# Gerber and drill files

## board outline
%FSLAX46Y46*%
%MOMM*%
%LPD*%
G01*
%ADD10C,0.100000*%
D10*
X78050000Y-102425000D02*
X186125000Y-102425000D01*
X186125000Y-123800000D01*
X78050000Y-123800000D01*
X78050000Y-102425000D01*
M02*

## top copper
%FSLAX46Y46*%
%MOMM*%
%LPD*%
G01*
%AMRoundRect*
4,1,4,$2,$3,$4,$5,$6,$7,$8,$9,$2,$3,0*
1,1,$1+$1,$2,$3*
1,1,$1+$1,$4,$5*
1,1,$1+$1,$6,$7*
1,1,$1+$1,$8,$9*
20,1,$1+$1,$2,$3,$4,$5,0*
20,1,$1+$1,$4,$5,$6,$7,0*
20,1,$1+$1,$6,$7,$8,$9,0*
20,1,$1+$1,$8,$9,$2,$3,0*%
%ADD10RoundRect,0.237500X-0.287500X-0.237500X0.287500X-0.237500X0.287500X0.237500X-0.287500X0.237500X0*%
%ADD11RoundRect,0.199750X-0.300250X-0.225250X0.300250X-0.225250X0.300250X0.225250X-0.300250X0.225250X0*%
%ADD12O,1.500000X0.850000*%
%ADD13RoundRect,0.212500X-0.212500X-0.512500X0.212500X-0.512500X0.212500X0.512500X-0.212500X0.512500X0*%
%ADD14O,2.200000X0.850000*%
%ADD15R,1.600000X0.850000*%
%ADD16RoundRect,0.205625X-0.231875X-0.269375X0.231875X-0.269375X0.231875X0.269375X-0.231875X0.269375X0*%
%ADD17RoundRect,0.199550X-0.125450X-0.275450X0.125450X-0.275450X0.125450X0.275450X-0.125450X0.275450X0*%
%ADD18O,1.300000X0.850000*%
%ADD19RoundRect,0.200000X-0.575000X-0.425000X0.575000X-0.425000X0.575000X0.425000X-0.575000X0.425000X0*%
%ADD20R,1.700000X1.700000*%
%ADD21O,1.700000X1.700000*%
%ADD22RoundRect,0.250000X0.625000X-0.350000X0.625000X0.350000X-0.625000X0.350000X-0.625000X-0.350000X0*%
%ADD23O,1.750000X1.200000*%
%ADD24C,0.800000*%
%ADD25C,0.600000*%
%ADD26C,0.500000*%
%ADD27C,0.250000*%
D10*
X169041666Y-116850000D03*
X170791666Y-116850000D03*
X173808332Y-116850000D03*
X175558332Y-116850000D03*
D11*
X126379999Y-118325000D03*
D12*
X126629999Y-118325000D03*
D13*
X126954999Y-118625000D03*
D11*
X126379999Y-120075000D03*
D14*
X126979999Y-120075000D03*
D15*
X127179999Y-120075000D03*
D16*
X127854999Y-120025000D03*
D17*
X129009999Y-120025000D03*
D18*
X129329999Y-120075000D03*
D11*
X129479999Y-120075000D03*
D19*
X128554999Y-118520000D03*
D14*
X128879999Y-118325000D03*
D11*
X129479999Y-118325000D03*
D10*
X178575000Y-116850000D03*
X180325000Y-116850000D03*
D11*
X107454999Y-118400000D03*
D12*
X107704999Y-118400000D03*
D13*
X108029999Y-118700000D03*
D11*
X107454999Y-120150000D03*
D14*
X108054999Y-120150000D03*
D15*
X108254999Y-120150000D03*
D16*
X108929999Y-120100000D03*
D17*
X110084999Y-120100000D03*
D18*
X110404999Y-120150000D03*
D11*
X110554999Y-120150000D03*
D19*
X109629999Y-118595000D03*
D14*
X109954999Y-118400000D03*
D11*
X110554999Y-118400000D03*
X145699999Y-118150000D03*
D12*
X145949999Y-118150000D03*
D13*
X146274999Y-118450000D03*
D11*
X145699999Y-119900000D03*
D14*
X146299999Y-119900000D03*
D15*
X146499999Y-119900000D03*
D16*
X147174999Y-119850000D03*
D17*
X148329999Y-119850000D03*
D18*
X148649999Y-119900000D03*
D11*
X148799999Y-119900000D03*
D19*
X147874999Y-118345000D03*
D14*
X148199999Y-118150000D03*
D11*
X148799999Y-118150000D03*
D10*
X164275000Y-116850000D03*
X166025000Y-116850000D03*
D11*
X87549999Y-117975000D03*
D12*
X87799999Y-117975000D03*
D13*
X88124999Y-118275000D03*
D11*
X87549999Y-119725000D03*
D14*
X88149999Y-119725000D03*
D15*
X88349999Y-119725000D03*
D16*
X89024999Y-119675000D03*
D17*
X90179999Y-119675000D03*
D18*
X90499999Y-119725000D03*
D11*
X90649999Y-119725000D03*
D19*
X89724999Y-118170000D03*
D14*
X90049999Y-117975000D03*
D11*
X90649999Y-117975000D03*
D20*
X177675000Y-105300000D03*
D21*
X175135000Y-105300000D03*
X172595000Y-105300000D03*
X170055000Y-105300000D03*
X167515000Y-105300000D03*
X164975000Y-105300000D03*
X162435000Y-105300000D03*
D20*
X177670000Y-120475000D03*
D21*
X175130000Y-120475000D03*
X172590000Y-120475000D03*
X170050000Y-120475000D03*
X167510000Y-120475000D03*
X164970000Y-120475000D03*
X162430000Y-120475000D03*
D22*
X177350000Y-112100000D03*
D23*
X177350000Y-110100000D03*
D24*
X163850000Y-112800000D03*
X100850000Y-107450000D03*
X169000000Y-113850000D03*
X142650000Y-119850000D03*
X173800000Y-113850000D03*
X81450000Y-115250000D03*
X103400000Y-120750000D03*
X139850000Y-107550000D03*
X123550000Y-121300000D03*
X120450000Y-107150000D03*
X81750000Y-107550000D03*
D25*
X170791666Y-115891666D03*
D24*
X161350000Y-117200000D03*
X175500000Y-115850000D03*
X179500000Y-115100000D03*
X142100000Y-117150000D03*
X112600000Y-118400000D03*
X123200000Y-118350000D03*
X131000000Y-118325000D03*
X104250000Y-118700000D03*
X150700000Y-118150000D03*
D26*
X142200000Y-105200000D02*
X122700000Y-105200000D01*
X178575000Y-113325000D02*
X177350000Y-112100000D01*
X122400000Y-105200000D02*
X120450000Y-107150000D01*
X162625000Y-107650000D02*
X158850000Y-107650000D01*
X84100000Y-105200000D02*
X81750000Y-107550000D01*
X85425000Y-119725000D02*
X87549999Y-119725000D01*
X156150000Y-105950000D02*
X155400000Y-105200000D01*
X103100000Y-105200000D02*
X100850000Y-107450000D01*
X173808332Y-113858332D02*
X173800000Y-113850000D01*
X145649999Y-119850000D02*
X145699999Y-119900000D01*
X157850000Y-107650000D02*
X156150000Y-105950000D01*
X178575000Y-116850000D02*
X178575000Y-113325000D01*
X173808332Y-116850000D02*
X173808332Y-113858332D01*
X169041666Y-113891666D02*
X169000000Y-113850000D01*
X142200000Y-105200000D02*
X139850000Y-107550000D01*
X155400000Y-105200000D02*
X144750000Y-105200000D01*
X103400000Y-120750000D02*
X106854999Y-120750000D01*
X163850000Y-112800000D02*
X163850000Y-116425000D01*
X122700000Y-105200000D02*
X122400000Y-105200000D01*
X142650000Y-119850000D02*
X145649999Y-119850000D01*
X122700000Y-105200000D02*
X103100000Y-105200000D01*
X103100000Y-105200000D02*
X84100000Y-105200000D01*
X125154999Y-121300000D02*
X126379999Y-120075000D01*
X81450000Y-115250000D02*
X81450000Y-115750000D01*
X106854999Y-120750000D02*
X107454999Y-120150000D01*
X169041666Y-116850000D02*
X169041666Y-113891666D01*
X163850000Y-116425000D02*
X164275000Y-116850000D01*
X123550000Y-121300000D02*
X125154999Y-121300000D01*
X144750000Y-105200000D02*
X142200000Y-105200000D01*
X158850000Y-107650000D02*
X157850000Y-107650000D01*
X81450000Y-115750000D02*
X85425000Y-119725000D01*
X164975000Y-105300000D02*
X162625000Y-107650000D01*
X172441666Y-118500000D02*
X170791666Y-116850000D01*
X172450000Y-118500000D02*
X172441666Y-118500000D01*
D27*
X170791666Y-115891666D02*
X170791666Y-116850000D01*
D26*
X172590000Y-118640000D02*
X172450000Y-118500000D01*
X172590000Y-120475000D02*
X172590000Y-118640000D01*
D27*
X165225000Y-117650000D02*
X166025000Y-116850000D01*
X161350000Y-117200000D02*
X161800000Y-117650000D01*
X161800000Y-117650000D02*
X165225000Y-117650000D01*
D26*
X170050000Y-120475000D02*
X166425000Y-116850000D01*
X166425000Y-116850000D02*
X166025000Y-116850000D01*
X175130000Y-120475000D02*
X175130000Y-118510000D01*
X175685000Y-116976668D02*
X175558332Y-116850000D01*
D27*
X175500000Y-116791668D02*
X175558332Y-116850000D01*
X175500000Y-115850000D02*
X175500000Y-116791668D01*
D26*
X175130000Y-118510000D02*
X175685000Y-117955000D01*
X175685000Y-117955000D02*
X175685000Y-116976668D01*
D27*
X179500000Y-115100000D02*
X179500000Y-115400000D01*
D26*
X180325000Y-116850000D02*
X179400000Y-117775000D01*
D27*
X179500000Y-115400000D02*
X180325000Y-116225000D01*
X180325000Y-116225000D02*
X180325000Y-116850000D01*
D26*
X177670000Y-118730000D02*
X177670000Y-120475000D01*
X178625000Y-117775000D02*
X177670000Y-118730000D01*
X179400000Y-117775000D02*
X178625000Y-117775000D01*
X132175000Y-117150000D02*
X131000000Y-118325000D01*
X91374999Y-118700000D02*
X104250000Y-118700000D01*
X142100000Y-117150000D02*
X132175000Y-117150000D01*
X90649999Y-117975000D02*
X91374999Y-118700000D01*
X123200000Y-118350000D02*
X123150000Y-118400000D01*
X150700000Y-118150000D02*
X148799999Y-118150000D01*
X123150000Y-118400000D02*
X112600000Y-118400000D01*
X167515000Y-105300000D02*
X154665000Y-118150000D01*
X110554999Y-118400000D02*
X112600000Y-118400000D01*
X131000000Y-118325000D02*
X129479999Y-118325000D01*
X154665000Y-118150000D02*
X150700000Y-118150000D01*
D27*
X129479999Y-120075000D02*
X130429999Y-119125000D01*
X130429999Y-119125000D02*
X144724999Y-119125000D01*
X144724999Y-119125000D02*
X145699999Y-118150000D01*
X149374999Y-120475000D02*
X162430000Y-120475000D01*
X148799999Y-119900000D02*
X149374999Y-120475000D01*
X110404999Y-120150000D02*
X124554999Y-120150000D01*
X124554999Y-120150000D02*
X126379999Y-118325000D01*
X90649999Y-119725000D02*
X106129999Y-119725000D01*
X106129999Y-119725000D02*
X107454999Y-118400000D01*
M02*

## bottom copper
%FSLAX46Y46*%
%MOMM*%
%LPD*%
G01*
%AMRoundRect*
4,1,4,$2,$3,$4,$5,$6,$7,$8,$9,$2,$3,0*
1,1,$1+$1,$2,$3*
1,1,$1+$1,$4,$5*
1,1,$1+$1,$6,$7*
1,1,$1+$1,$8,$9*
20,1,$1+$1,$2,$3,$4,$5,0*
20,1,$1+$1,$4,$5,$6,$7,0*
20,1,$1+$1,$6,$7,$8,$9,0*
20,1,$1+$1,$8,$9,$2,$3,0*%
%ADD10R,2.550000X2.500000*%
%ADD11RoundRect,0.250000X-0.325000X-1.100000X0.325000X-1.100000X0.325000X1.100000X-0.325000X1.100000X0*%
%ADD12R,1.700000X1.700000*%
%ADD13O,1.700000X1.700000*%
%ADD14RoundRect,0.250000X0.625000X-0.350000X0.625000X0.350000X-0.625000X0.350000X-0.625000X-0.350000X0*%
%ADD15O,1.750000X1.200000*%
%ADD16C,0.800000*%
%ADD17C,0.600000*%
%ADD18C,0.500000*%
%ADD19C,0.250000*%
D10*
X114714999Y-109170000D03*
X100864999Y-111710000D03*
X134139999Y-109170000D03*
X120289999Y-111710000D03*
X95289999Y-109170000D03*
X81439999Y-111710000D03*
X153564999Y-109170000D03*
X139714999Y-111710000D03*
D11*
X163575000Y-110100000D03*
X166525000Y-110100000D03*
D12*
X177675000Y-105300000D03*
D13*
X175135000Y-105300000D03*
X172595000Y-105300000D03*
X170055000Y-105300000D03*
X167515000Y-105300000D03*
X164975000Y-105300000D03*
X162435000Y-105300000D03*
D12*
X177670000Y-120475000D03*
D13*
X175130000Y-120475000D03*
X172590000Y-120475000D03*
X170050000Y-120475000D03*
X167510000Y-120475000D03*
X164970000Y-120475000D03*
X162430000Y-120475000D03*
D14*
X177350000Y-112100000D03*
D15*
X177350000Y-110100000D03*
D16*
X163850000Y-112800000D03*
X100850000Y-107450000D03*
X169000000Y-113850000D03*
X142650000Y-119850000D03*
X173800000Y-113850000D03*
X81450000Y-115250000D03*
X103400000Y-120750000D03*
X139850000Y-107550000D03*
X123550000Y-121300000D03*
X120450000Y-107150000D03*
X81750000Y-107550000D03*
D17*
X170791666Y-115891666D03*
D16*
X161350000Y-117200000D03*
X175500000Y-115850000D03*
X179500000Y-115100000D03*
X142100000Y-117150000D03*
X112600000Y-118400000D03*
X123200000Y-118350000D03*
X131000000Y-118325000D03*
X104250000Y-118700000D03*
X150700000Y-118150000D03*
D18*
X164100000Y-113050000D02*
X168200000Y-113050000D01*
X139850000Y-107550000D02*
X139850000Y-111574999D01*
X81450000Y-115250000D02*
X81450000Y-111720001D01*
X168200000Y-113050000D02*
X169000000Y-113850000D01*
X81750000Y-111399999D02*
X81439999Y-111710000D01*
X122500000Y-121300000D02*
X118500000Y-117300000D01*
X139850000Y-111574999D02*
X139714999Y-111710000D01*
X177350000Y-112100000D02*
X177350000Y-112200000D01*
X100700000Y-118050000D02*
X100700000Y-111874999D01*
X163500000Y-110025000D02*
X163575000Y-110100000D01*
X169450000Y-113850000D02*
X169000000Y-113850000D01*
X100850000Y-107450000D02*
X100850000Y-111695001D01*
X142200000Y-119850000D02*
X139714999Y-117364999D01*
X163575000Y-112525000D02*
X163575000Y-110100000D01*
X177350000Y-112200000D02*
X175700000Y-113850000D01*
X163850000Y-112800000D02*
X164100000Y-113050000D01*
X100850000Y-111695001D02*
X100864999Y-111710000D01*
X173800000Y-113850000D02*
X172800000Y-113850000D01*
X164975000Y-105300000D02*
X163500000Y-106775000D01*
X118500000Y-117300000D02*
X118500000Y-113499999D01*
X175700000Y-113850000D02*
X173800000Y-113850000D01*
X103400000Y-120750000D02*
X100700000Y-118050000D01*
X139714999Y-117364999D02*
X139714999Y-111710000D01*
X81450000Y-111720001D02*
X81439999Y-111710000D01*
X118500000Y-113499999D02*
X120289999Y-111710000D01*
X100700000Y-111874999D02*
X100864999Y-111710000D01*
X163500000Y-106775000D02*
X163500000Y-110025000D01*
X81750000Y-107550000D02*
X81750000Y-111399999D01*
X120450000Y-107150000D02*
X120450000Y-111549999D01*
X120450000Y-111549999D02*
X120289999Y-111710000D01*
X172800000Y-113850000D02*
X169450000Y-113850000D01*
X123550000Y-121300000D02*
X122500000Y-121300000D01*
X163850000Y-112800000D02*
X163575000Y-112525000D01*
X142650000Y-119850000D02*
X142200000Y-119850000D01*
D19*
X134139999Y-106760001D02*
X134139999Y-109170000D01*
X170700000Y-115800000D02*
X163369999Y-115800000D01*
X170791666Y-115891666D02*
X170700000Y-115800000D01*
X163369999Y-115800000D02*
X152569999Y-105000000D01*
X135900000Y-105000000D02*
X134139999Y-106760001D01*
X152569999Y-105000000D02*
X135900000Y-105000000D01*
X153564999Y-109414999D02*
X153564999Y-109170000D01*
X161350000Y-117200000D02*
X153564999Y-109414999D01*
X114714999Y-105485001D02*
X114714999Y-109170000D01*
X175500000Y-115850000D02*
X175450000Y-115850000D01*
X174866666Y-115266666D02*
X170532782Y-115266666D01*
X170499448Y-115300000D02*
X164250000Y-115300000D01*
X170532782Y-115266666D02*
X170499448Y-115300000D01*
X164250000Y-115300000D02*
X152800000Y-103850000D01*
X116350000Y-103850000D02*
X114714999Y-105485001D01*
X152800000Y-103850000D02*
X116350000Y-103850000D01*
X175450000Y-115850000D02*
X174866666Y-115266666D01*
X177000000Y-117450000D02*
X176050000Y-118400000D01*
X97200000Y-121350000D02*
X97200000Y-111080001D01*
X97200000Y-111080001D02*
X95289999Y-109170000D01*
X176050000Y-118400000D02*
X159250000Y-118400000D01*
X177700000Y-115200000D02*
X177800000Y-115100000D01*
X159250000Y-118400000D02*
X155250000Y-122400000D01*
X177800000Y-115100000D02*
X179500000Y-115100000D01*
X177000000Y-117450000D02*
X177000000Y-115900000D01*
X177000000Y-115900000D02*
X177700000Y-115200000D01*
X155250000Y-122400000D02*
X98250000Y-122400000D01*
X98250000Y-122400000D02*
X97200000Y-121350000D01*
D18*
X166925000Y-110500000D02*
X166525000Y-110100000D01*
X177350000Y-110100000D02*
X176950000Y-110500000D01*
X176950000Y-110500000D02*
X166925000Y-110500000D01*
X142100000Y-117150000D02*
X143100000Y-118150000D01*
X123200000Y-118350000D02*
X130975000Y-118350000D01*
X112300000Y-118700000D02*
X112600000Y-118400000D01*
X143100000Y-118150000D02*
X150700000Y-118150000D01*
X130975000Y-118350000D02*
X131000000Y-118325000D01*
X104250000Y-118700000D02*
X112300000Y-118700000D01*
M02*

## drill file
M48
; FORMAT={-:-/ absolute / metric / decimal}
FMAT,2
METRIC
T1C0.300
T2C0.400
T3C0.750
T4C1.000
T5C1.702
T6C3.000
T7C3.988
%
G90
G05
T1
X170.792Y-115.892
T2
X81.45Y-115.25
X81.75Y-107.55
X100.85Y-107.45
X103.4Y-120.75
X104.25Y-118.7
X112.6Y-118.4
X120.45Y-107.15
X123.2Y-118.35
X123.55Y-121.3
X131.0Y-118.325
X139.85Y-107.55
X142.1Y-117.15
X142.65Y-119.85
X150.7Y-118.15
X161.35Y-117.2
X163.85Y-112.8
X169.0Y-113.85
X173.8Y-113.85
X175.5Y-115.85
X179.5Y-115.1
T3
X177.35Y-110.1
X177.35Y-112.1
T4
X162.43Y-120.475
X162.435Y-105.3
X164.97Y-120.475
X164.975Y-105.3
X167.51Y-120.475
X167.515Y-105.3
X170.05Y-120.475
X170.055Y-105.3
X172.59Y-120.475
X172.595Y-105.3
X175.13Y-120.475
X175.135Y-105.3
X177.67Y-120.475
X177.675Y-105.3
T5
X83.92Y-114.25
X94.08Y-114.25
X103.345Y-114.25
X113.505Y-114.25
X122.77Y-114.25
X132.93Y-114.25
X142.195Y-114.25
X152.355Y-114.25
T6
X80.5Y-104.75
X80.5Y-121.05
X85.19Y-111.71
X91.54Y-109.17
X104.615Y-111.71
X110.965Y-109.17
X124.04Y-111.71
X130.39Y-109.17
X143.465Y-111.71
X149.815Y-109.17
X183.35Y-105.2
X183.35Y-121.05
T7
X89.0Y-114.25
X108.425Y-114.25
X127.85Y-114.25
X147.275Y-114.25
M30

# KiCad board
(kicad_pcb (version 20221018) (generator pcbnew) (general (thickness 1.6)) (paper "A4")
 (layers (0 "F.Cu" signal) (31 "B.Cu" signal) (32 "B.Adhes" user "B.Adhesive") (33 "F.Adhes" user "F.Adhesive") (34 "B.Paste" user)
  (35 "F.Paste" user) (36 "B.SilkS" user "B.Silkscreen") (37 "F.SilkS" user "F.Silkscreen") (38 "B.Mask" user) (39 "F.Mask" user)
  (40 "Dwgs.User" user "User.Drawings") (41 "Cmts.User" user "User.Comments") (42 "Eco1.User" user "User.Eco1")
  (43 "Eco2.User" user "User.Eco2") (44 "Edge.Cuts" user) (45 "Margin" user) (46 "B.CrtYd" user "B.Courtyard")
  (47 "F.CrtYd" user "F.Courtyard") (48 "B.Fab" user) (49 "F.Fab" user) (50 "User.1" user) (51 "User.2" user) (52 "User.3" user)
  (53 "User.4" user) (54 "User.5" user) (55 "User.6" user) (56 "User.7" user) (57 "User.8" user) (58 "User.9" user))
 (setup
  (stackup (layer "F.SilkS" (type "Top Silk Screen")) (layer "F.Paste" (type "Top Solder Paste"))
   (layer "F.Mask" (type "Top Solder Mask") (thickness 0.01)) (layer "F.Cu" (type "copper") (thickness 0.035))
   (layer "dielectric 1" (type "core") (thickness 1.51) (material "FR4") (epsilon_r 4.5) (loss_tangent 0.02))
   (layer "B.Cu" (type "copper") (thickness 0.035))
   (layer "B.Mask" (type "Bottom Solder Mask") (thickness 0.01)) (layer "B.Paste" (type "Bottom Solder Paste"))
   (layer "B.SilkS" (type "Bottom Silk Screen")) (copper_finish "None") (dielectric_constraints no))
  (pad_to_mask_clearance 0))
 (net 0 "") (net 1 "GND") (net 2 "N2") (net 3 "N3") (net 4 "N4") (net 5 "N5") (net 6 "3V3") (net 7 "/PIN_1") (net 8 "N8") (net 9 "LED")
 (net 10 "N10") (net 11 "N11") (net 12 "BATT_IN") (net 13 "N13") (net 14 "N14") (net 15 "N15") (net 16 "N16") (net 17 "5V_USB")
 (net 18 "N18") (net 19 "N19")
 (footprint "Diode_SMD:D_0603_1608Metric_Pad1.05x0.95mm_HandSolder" (layer "F.Cu") (at 169.916666 116.85)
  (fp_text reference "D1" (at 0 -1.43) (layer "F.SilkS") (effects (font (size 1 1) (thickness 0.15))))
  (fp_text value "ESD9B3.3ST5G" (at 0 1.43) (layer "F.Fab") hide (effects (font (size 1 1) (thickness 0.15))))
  (pad "1" smd roundrect (at -0.875 0) (size 1.05 0.95) (layers "F.Cu" "F.Paste" "F.Mask") (roundrect_rratio 0.25) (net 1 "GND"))
  (pad "2" smd roundrect (at 0.875 0) (size 1.05 0.95) (layers "F.Cu" "F.Paste" "F.Mask") (roundrect_rratio 0.25) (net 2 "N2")))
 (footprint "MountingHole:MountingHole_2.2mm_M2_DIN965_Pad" (layer "F.Cu") (at 183.35 121.05)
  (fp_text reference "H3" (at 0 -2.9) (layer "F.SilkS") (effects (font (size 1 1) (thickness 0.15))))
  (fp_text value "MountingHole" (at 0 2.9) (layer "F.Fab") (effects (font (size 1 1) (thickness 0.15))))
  (pad "" np_thru_hole circle (at 0 0) (size 3 3) (drill 3) (layers "F&B.Cu" "*.Mask")))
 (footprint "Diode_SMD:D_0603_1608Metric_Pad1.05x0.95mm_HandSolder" (layer "F.Cu") (at 174.683332 116.85)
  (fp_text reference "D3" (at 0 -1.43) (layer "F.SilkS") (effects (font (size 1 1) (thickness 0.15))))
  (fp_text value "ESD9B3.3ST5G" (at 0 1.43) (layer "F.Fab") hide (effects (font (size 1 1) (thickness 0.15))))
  (pad "1" smd roundrect (at -0.875 0) (size 1.05 0.95) (layers "F.Cu" "F.Paste" "F.Mask") (roundrect_rratio 0.25) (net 1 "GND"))
  (pad "2" smd roundrect (at 0.875 0) (size 1.05 0.95) (layers "F.Cu" "F.Paste" "F.Mask") (roundrect_rratio 0.25) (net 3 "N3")))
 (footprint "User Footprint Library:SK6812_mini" (layer "F.Cu") (at 127.929999 119.2) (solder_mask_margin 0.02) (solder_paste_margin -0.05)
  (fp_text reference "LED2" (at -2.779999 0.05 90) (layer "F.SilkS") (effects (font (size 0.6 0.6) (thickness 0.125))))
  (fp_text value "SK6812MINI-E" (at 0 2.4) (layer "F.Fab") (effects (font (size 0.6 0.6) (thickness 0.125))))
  (pad "1" smd roundrect (at -1.55 -0.875) (size 1 0.85) (layers "F.Cu" "F.Mask") (roundrect_rratio 0.235) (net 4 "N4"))
  (pad "1" smd oval (at -1.3 -0.875) (size 1.5 0.85) (layers "F.Cu" "F.Paste") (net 4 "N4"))
  (pad "1" smd roundrect (at -0.975 -0.575) (size 0.85 1.45) (layers "F.Cu" "F.Mask") (roundrect_rratio 0.25) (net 4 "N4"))
  (pad "2" smd roundrect (at -1.55 0.875) (size 1 0.85) (layers "F.Cu" "F.Mask") (roundrect_rratio 0.235) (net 1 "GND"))
  (pad "2" smd oval (at -0.95 0.875) (size 2.2 0.85) (layers "F.Cu" "F.Paste") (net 1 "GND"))
  (pad "2" smd rect (at -0.75 0.875) (size 1.6 0.85) (layers "F.Cu" "F.Mask") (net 1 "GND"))
  (pad "2" smd roundrect (at -0.075 0.825) (size 0.875 0.95) (layers "F.Cu" "F.Mask") (roundrect_rratio 0.235) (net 1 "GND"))
  (pad "3" smd roundrect (at 1.08 0.825) (size 0.65 0.95) (layers "F.Cu" "F.Mask") (roundrect_rratio 0.307) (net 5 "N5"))
  (pad "3" smd oval (at 1.4 0.875) (size 1.3 0.85) (layers "F.Cu" "F.Paste") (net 5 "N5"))
  (pad "3" smd roundrect (at 1.55 0.875) (size 1 0.85) (layers "F.Cu" "F.Mask") (roundrect_rratio 0.235) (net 5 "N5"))
  (pad "4" smd roundrect (at 0.625 -0.68) (size 1.55 1.25) (layers "F.Cu" "F.Mask") (roundrect_rratio 0.16) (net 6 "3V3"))
  (pad "4" smd oval (at 0.95 -0.875) (size 2.2 0.85) (layers "F.Cu" "F.Paste") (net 6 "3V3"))
  (pad "4" smd roundrect (at 1.55 -0.875) (size 1 0.85) (layers "F.Cu" "F.Mask") (roundrect_rratio 0.235) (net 6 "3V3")))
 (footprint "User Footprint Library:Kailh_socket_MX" (layer "F.Cu") (at 108.424999 114.25)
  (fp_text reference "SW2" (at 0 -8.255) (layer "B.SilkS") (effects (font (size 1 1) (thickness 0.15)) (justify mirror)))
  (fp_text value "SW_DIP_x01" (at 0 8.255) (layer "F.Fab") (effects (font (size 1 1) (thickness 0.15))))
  (pad "" np_thru_hole circle (at -5.08 0) (size 1.7018 1.7018) (drill 1.7018) (layers "*.Cu" "*.Mask"))
  (pad "" np_thru_hole circle (at -3.81 -2.54) (size 3 3) (drill 3) (layers "*.Cu" "*.Mask"))
  (pad "" np_thru_hole circle (at 0 0) (size 3.9878 3.9878) (drill 3.9878) (layers "*.Cu" "*.Mask"))
  (pad "" np_thru_hole circle (at 2.54 -5.08) (size 3 3) (drill 3) (layers "*.Cu" "*.Mask"))
  (pad "" np_thru_hole circle (at 5.08 0) (size 1.7018 1.7018) (drill 1.7018) (layers "*.Cu" "*.Mask"))
  (pad "1" smd rect (at 6.29 -5.08) (size 2.55 2.5) (layers "B.Cu" "B.Paste" "B.Mask") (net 3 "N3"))
  (pad "2" smd rect (at -7.56 -2.54) (size 2.55 2.5) (layers "B.Cu" "B.Paste" "B.Mask") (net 1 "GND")))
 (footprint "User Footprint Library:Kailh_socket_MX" (layer "F.Cu") (at 127.849999 114.25)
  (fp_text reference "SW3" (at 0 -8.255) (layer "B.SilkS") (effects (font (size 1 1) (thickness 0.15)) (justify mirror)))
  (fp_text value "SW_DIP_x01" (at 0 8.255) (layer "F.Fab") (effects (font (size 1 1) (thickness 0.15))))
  (pad "" np_thru_hole circle (at -5.08 0) (size 1.7018 1.7018) (drill 1.7018) (layers "*.Cu" "*.Mask"))
  (pad "" np_thru_hole circle (at -3.81 -2.54) (size 3 3) (drill 3) (layers "*.Cu" "*.Mask"))
  (pad "" np_thru_hole circle (at 0 0) (size 3.9878 3.9878) (drill 3.9878) (layers "*.Cu" "*.Mask"))
  (pad "" np_thru_hole circle (at 2.54 -5.08) (size 3 3) (drill 3) (layers "*.Cu" "*.Mask"))
  (pad "" np_thru_hole circle (at 5.08 0) (size 1.7018 1.7018) (drill 1.7018) (layers "*.Cu" "*.Mask"))
  (pad "1" smd rect (at 6.29 -5.08) (size 2.55 2.5) (layers "B.Cu" "B.Paste" "B.Mask") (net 2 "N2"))
  (pad "2" smd rect (at -7.56 -2.54) (size 2.55 2.5) (layers "B.Cu" "B.Paste" "B.Mask") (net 1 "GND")))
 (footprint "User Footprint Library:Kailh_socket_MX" (layer "F.Cu") (at 88.999999 114.25)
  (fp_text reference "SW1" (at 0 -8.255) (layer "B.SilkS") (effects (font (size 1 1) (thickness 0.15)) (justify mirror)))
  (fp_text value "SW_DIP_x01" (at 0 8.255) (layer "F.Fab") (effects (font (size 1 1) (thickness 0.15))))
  (pad "" np_thru_hole circle (at -5.08 0) (size 1.7018 1.7018) (drill 1.7018) (layers "*.Cu" "*.Mask"))
  (pad "" np_thru_hole circle (at -3.81 -2.54) (size 3 3) (drill 3) (layers "*.Cu" "*.Mask"))
  (pad "" np_thru_hole circle (at 0 0) (size 3.9878 3.9878) (drill 3.9878) (layers "*.Cu" "*.Mask"))
  (pad "" np_thru_hole circle (at 2.54 -5.08) (size 3 3) (drill 3) (layers "*.Cu" "*.Mask"))
  (pad "" np_thru_hole circle (at 5.08 0) (size 1.7018 1.7018) (drill 1.7018) (layers "*.Cu" "*.Mask"))
  (pad "1" smd rect (at 6.29 -5.08) (size 2.55 2.5) (layers "B.Cu" "B.Paste" "B.Mask") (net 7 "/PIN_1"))
  (pad "2" smd rect (at -7.56 -2.54) (size 2.55 2.5) (layers "B.Cu" "B.Paste" "B.Mask") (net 1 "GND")))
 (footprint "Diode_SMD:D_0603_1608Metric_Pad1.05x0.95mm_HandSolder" (layer "F.Cu") (at 179.45 116.85)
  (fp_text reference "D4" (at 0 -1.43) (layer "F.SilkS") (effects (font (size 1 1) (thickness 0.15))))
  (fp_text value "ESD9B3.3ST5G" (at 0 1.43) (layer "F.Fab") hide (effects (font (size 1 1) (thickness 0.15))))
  (pad "1" smd roundrect (at -0.875 0) (size 1.05 0.95) (layers "F.Cu" "F.Paste" "F.Mask") (roundrect_rratio 0.25) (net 1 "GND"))
  (pad "2" smd roundrect (at 0.875 0) (size 1.05 0.95) (layers "F.Cu" "F.Paste" "F.Mask") (roundrect_rratio 0.25) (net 7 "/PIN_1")))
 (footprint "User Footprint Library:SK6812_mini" (layer "F.Cu") (at 109.004999 119.275) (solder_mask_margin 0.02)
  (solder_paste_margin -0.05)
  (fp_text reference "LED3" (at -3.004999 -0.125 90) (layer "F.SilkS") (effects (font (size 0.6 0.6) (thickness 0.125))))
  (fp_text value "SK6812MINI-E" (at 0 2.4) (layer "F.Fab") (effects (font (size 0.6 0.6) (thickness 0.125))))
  (pad "1" smd roundrect (at -1.55 -0.875) (size 1 0.85) (layers "F.Cu" "F.Mask") (roundrect_rratio 0.235) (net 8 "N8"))
  (pad "1" smd oval (at -1.3 -0.875) (size 1.5 0.85) (layers "F.Cu" "F.Paste") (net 8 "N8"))
  (pad "1" smd roundrect (at -0.975 -0.575) (size 0.85 1.45) (layers "F.Cu" "F.Mask") (roundrect_rratio 0.25) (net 8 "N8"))
  (pad "2" smd roundrect (at -1.55 0.875) (size 1 0.85) (layers "F.Cu" "F.Mask") (roundrect_rratio 0.235) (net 1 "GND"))
  (pad "2" smd oval (at -0.95 0.875) (size 2.2 0.85) (layers "F.Cu" "F.Paste") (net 1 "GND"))
  (pad "2" smd rect (at -0.75 0.875) (size 1.6 0.85) (layers "F.Cu" "F.Mask") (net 1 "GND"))
  (pad "2" smd roundrect (at -0.075 0.825) (size 0.875 0.95) (layers "F.Cu" "F.Mask") (roundrect_rratio 0.235) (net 1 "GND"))
  (pad "3" smd roundrect (at 1.08 0.825) (size 0.65 0.95) (layers "F.Cu" "F.Mask") (roundrect_rratio 0.307) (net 4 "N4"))
  (pad "3" smd oval (at 1.4 0.875) (size 1.3 0.85) (layers "F.Cu" "F.Paste") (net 4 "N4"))
  (pad "3" smd roundrect (at 1.55 0.875) (size 1 0.85) (layers "F.Cu" "F.Mask") (roundrect_rratio 0.235) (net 4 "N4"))
  (pad "4" smd roundrect (at 0.625 -0.68) (size 1.55 1.25) (layers "F.Cu" "F.Mask") (roundrect_rratio 0.16) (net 6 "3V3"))
  (pad "4" smd oval (at 0.95 -0.875) (size 2.2 0.85) (layers "F.Cu" "F.Paste") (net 6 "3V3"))
  (pad "4" smd roundrect (at 1.55 -0.875) (size 1 0.85) (layers "F.Cu" "F.Mask") (roundrect_rratio 0.235) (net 6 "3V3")))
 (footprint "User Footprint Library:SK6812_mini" (layer "F.Cu") (at 147.249999 119.025) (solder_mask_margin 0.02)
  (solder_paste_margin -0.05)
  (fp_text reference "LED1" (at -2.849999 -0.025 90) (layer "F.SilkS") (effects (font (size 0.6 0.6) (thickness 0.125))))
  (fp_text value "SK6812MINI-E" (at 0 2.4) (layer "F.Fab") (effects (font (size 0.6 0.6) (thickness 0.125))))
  (pad "1" smd roundrect (at -1.55 -0.875) (size 1 0.85) (layers "F.Cu" "F.Mask") (roundrect_rratio 0.235) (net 5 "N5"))
  (pad "1" smd oval (at -1.3 -0.875) (size 1.5 0.85) (layers "F.Cu" "F.Paste") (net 5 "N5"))
  (pad "1" smd roundrect (at -0.975 -0.575) (size 0.85 1.45) (layers "F.Cu" "F.Mask") (roundrect_rratio 0.25) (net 5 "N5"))
  (pad "2" smd roundrect (at -1.55 0.875) (size 1 0.85) (layers "F.Cu" "F.Mask") (roundrect_rratio 0.235) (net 1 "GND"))
  (pad "2" smd oval (at -0.95 0.875) (size 2.2 0.85) (layers "F.Cu" "F.Paste") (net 1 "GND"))
  (pad "2" smd rect (at -0.75 0.875) (size 1.6 0.85) (layers "F.Cu" "F.Mask") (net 1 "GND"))
  (pad "2" smd roundrect (at -0.075 0.825) (size 0.875 0.95) (layers "F.Cu" "F.Mask") (roundrect_rratio 0.235) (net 1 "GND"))
  (pad "3" smd roundrect (at 1.08 0.825) (size 0.65 0.95) (layers "F.Cu" "F.Mask") (roundrect_rratio 0.307) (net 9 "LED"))
  (pad "3" smd oval (at 1.4 0.875) (size 1.3 0.85) (layers "F.Cu" "F.Paste") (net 9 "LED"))
  (pad "3" smd roundrect (at 1.55 0.875) (size 1 0.85) (layers "F.Cu" "F.Mask") (roundrect_rratio 0.235) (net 9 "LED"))
  (pad "4" smd roundrect (at 0.625 -0.68) (size 1.55 1.25) (layers "F.Cu" "F.Mask") (roundrect_rratio 0.16) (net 6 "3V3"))
  (pad "4" smd oval (at 0.95 -0.875) (size 2.2 0.85) (layers "F.Cu" "F.Paste") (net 6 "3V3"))
  (pad "4" smd roundrect (at 1.55 -0.875) (size 1 0.85) (layers "F.Cu" "F.Mask") (roundrect_rratio 0.235) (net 6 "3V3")))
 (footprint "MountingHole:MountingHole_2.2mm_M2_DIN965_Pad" (layer "F.Cu") (at 183.35 105.2)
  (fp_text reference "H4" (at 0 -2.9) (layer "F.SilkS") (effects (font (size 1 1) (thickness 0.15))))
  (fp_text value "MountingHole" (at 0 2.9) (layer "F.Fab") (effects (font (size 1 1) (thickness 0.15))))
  (pad "" np_thru_hole circle (at 0 0) (size 3 3) (drill 3) (layers "F&B.Cu" "*.Mask")))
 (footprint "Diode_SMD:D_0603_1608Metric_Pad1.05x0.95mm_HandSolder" (layer "F.Cu") (at 165.15 116.85)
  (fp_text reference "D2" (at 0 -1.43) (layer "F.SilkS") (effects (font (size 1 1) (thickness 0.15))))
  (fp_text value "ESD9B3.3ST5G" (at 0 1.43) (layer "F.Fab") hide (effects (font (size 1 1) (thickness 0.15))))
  (pad "1" smd roundrect (at -0.875 0) (size 1.05 0.95) (layers "F.Cu" "F.Paste" "F.Mask") (roundrect_rratio 0.25) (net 1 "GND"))
  (pad "2" smd roundrect (at 0.875 0) (size 1.05 0.95) (layers "F.Cu" "F.Paste" "F.Mask") (roundrect_rratio 0.25) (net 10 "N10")))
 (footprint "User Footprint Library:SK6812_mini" (layer "F.Cu") (at 89.099999 118.85) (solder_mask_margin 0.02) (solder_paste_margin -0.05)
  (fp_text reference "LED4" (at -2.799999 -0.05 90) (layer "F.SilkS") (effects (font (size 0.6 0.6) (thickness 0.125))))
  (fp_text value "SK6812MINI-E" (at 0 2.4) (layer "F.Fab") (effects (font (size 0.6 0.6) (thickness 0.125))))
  (pad "1" smd roundrect (at -1.55 -0.875) (size 1 0.85) (layers "F.Cu" "F.Mask") (roundrect_rratio 0.235) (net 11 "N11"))
  (pad "1" smd oval (at -1.3 -0.875) (size 1.5 0.85) (layers "F.Cu" "F.Paste") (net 11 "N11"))
  (pad "1" smd roundrect (at -0.975 -0.575) (size 0.85 1.45) (layers "F.Cu" "F.Mask") (roundrect_rratio 0.25) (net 11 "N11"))
  (pad "2" smd roundrect (at -1.55 0.875) (size 1 0.85) (layers "F.Cu" "F.Mask") (roundrect_rratio 0.235) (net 1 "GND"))
  (pad "2" smd oval (at -0.95 0.875) (size 2.2 0.85) (layers "F.Cu" "F.Paste") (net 1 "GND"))
  (pad "2" smd rect (at -0.75 0.875) (size 1.6 0.85) (layers "F.Cu" "F.Mask") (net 1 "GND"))
  (pad "2" smd roundrect (at -0.075 0.825) (size 0.875 0.95) (layers "F.Cu" "F.Mask") (roundrect_rratio 0.235) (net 1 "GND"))
  (pad "3" smd roundrect (at 1.08 0.825) (size 0.65 0.95) (layers "F.Cu" "F.Mask") (roundrect_rratio 0.307) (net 8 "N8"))
  (pad "3" smd oval (at 1.4 0.875) (size 1.3 0.85) (layers "F.Cu" "F.Paste") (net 8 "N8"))
  (pad "3" smd roundrect (at 1.55 0.875) (size 1 0.85) (layers "F.Cu" "F.Mask") (roundrect_rratio 0.235) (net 8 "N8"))
  (pad "4" smd roundrect (at 0.625 -0.68) (size 1.55 1.25) (layers "F.Cu" "F.Mask") (roundrect_rratio 0.16) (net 6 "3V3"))
  (pad "4" smd oval (at 0.95 -0.875) (size 2.2 0.85) (layers "F.Cu" "F.Paste") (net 6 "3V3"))
  (pad "4" smd roundrect (at 1.55 -0.875) (size 1 0.85) (layers "F.Cu" "F.Mask") (roundrect_rratio 0.235) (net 6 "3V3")))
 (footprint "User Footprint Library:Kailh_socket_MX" (layer "F.Cu") (at 147.274999 114.25)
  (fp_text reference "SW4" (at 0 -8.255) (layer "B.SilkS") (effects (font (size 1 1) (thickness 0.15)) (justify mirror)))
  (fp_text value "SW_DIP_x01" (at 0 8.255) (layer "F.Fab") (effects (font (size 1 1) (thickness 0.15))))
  (pad "" np_thru_hole circle (at -5.08 0) (size 1.7018 1.7018) (drill 1.7018) (layers "*.Cu" "*.Mask"))
  (pad "" np_thru_hole circle (at -3.81 -2.54) (size 3 3) (drill 3) (layers "*.Cu" "*.Mask"))
  (pad "" np_thru_hole circle (at 0 0) (size 3.9878 3.9878) (drill 3.9878) (layers "*.Cu" "*.Mask"))
  (pad "" np_thru_hole circle (at 2.54 -5.08) (size 3 3) (drill 3) (layers "*.Cu" "*.Mask"))
  (pad "" np_thru_hole circle (at 5.08 0) (size 1.7018 1.7018) (drill 1.7018) (layers "*.Cu" "*.Mask"))
  (pad "1" smd rect (at 6.29 -5.08) (size 2.55 2.5) (layers "B.Cu" "B.Paste" "B.Mask") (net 10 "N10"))
  (pad "2" smd rect (at -7.56 -2.54) (size 2.55 2.5) (layers "B.Cu" "B.Paste" "B.Mask") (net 1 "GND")))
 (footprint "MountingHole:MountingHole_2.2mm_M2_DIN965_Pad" (layer "F.Cu") (at 80.5 121.05)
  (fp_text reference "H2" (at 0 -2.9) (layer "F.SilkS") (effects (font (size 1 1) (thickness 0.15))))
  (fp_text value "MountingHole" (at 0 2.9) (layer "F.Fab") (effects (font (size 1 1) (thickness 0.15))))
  (pad "" np_thru_hole circle (at 0 0) (size 3 3) (drill 3) (layers "F&B.Cu" "*.Mask")))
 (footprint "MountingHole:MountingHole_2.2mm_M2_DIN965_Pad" (layer "F.Cu") (at 80.5 104.75)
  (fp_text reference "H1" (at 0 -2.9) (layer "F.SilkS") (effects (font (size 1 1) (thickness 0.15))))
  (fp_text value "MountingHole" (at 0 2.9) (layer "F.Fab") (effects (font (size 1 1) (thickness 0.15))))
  (pad "" np_thru_hole circle (at 0 0) (size 3 3) (drill 3) (layers "F&B.Cu" "*.Mask")))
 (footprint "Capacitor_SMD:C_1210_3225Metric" (layer "B.Cu") (at 165.05 110.1)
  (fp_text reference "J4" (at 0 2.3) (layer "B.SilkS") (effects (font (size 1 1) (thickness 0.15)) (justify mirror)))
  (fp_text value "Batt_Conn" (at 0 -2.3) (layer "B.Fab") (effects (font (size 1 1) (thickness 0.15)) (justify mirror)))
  (pad "1" smd roundrect (at -1.475 0) (size 1.15 2.7) (layers "B.Cu" "B.Paste" "B.Mask") (roundrect_rratio 0.217391) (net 1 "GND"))
  (pad "2" smd roundrect (at 1.475 0) (size 1.15 2.7) (layers "B.Cu" "B.Paste" "B.Mask") (roundrect_rratio 0.217391) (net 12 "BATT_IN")))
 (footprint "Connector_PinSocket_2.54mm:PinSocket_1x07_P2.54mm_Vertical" (layer "B.Cu") (at 177.675 105.3 90)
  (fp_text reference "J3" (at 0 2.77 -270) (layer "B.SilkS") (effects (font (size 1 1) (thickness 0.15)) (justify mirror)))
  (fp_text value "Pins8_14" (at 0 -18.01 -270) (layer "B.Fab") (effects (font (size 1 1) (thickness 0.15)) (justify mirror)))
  (pad "1" thru_hole rect (at 0 0 90) (size 1.7 1.7) (drill 1) (layers "*.Cu" "*.Mask") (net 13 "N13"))
  (pad "2" thru_hole oval (at 0 -2.54 90) (size 1.7 1.7) (drill 1) (layers "*.Cu" "*.Mask") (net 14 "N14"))
  (pad "3" thru_hole oval (at 0 -5.08 90) (size 1.7 1.7) (drill 1) (layers "*.Cu" "*.Mask") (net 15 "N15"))
  (pad "4" thru_hole oval (at 0 -7.62 90) (size 1.7 1.7) (drill 1) (layers "*.Cu" "*.Mask") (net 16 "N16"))
  (pad "5" thru_hole oval (at 0 -10.16 90) (size 1.7 1.7) (drill 1) (layers "*.Cu" "*.Mask") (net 6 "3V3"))
  (pad "6" thru_hole oval (at 0 -12.7 90) (size 1.7 1.7) (drill 1) (layers "*.Cu" "*.Mask") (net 1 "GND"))
  (pad "7" thru_hole oval (at 0 -15.24 90) (size 1.7 1.7) (drill 1) (layers "*.Cu" "*.Mask") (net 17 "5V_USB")))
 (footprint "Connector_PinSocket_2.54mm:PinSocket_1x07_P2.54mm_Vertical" (layer "B.Cu") (at 177.67 120.475 90)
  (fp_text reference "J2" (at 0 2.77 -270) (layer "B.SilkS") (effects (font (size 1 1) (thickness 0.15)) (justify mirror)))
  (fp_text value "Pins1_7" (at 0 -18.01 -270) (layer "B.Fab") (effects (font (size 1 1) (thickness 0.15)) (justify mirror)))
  (pad "1" thru_hole rect (at 0 0 90) (size 1.7 1.7) (drill 1) (layers "*.Cu" "*.Mask") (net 7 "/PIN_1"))
  (pad "2" thru_hole oval (at 0 -2.54 90) (size 1.7 1.7) (drill 1) (layers "*.Cu" "*.Mask") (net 3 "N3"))
  (pad "3" thru_hole oval (at 0 -5.08 90) (size 1.7 1.7) (drill 1) (layers "*.Cu" "*.Mask") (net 2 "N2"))
  (pad "4" thru_hole oval (at 0 -7.62 90) (size 1.7 1.7) (drill 1) (layers "*.Cu" "*.Mask") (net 10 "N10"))
  (pad "5" thru_hole oval (at 0 -10.16 90) (size 1.7 1.7) (drill 1) (layers "*.Cu" "*.Mask") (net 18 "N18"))
  (pad "6" thru_hole oval (at 0 -12.7 90) (size 1.7 1.7) (drill 1) (layers "*.Cu" "*.Mask") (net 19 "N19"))
  (pad "7" thru_hole oval (at 0 -15.24 90) (size 1.7 1.7) (drill 1) (layers "*.Cu" "*.Mask") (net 9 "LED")))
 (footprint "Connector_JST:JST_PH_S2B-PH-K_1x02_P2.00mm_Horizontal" (layer "B.Cu") (at 177.35 112.1 90)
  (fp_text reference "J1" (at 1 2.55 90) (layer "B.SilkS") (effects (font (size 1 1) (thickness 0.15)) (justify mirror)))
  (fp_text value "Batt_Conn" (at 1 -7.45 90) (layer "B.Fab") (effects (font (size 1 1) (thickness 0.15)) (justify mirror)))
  (pad "1" thru_hole roundrect (at 0 0 90) (size 1.2 1.75) (drill 0.75) (layers "*.Cu" "*.Mask") (roundrect_rratio 0.208333) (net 1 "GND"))
  (pad "2" thru_hole oval (at 2 0 90) (size 1.2 1.75) (drill 0.75) (layers "*.Cu" "*.Mask") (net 12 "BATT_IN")))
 (gr_rect (start 78.05 102.425) (end 186.125 123.8) (stroke (width 0.1) (type default)) (fill none) (layer "Edge.Cuts"))
 (segment (start 142.2 105.2) (end 122.7 105.2) (width 0.5) (layer "F.Cu") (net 1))
 (segment (start 178.575 113.325) (end 177.35 112.1) (width 0.5) (layer "F.Cu") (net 1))
 (segment (start 122.4 105.2) (end 120.45 107.15) (width 0.5) (layer "F.Cu") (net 1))
 (segment (start 162.625 107.65) (end 158.85 107.65) (width 0.5) (layer "F.Cu") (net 1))
 (segment (start 84.1 105.2) (end 81.75 107.55) (width 0.5) (layer "F.Cu") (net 1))
 (segment (start 85.425 119.725) (end 87.549999 119.725) (width 0.5) (layer "F.Cu") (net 1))
 (segment (start 156.15 105.95) (end 155.4 105.2) (width 0.5) (layer "F.Cu") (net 1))
 (segment (start 103.1 105.2) (end 100.85 107.45) (width 0.5) (layer "F.Cu") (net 1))
 (segment (start 173.808332 113.858332) (end 173.8 113.85) (width 0.5) (layer "F.Cu") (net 1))
 (segment (start 145.649999 119.85) (end 145.699999 119.9) (width 0.5) (layer "F.Cu") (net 1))
 (segment (start 157.85 107.65) (end 156.15 105.95) (width 0.5) (layer "F.Cu") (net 1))
 (segment (start 178.575 116.85) (end 178.575 113.325) (width 0.5) (layer "F.Cu") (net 1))
 (segment (start 173.808332 116.85) (end 173.808332 113.858332) (width 0.5) (layer "F.Cu") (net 1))
 (segment (start 169.041666 113.891666) (end 169 113.85) (width 0.5) (layer "F.Cu") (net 1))
 (segment (start 142.2 105.2) (end 139.85 107.55) (width 0.5) (layer "F.Cu") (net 1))
 (segment (start 155.4 105.2) (end 144.75 105.2) (width 0.5) (layer "F.Cu") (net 1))
 (segment (start 103.4 120.75) (end 106.854999 120.75) (width 0.5) (layer "F.Cu") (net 1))
 (segment (start 163.85 112.8) (end 163.85 116.425) (width 0.5) (layer "F.Cu") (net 1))
 (segment (start 122.7 105.2) (end 122.4 105.2) (width 0.5) (layer "F.Cu") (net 1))
 (segment (start 142.65 119.85) (end 145.649999 119.85) (width 0.5) (layer "F.Cu") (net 1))
 (segment (start 122.7 105.2) (end 103.1 105.2) (width 0.5) (layer "F.Cu") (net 1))
 (segment (start 103.1 105.2) (end 84.1 105.2) (width 0.5) (layer "F.Cu") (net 1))
 (segment (start 125.154999 121.3) (end 126.379999 120.075) (width 0.5) (layer "F.Cu") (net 1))
 (segment (start 81.45 115.25) (end 81.45 115.75) (width 0.5) (layer "F.Cu") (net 1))
 (segment (start 106.854999 120.75) (end 107.454999 120.15) (width 0.5) (layer "F.Cu") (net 1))
 (segment (start 169.041666 116.85) (end 169.041666 113.891666) (width 0.5) (layer "F.Cu") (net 1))
 (segment (start 163.85 116.425) (end 164.275 116.85) (width 0.5) (layer "F.Cu") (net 1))
 (segment (start 123.55 121.3) (end 125.154999 121.3) (width 0.5) (layer "F.Cu") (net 1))
 (segment (start 144.75 105.2) (end 142.2 105.2) (width 0.5) (layer "F.Cu") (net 1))
 (segment (start 158.85 107.65) (end 157.85 107.65) (width 0.5) (layer "F.Cu") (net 1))
 (segment (start 81.45 115.75) (end 85.425 119.725) (width 0.5) (layer "F.Cu") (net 1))
 (segment (start 164.975 105.3) (end 162.625 107.65) (width 0.5) (layer "F.Cu") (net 1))
 (via (at 163.85 112.8) (size 0.8) (drill 0.4) (layers "F.Cu" "B.Cu") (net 1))
 (via (at 100.85 107.45) (size 0.8) (drill 0.4) (layers "F.Cu" "B.Cu") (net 1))
 (via (at 169 113.85) (size 0.8) (drill 0.4) (layers "F.Cu" "B.Cu") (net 1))
 (via (at 142.65 119.85) (size 0.8) (drill 0.4) (layers "F.Cu" "B.Cu") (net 1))
 (via (at 173.8 113.85) (size 0.8) (drill 0.4) (layers "F.Cu" "B.Cu") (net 1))
 (via (at 81.45 115.25) (size 0.8) (drill 0.4) (layers "F.Cu" "B.Cu") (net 1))
 (via (at 103.4 120.75) (size 0.8) (drill 0.4) (layers "F.Cu" "B.Cu") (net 1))
 (via (at 139.85 107.55) (size 0.8) (drill 0.4) (layers "F.Cu" "B.Cu") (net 1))
 (via (at 123.55 121.3) (size 0.8) (drill 0.4) (layers "F.Cu" "B.Cu") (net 1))
 (via (at 120.45 107.15) (size 0.8) (drill 0.4) (layers "F.Cu" "B.Cu") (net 1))
 (via (at 81.75 107.55) (size 0.8) (drill 0.4) (layers "F.Cu" "B.Cu") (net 1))
 (segment (start 164.1 113.05) (end 168.2 113.05) (width 0.5) (layer "B.Cu") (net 1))
 (segment (start 139.85 107.55) (end 139.85 111.574999) (width 0.5) (layer "B.Cu") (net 1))
 (segment (start 81.45 115.25) (end 81.45 111.720001) (width 0.5) (layer "B.Cu") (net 1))
 (segment (start 168.2 113.05) (end 169 113.85) (width 0.5) (layer "B.Cu") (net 1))
 (segment (start 81.75 111.399999) (end 81.439999 111.71) (width 0.5) (layer "B.Cu") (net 1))
 (segment (start 122.5 121.3) (end 118.5 117.3) (width 0.5) (layer "B.Cu") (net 1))
 (segment (start 139.85 111.574999) (end 139.714999 111.71) (width 0.5) (layer "B.Cu") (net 1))
 (segment (start 177.35 112.1) (end 177.35 112.2) (width 0.5) (layer "B.Cu") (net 1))
 (segment (start 100.7 118.05) (end 100.7 111.874999) (width 0.5) (layer "B.Cu") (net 1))
 (segment (start 163.5 110.025) (end 163.575 110.1) (width 0.5) (layer "B.Cu") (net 1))
 (segment (start 169.45 113.85) (end 169 113.85) (width 0.5) (layer "B.Cu") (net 1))
 (segment (start 100.85 107.45) (end 100.85 111.695001) (width 0.5) (layer "B.Cu") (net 1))
 (segment (start 142.2 119.85) (end 139.714999 117.364999) (width 0.5) (layer "B.Cu") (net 1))
 (segment (start 163.575 112.525) (end 163.575 110.1) (width 0.5) (layer "B.Cu") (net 1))
 (segment (start 177.35 112.2) (end 175.7 113.85) (width 0.5) (layer "B.Cu") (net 1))
 (segment (start 163.85 112.8) (end 164.1 113.05) (width 0.5) (layer "B.Cu") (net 1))
 (segment (start 100.85 111.695001) (end 100.864999 111.71) (width 0.5) (layer "B.Cu") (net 1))
 (segment (start 173.8 113.85) (end 172.8 113.85) (width 0.5) (layer "B.Cu") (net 1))
 (segment (start 164.975 105.3) (end 163.5 106.775) (width 0.5) (layer "B.Cu") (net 1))
 (segment (start 118.5 117.3) (end 118.5 113.499999) (width 0.5) (layer "B.Cu") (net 1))
 (segment (start 175.7 113.85) (end 173.8 113.85) (width 0.5) (layer "B.Cu") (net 1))
 (segment (start 103.4 120.75) (end 100.7 118.05) (width 0.5) (layer "B.Cu") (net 1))
 (segment (start 139.714999 117.364999) (end 139.714999 111.71) (width 0.5) (layer "B.Cu") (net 1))
 (segment (start 81.45 111.720001) (end 81.439999 111.71) (width 0.5) (layer "B.Cu") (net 1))
 (segment (start 118.5 113.499999) (end 120.289999 111.71) (width 0.5) (layer "B.Cu") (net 1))
 (segment (start 100.7 111.874999) (end 100.864999 111.71) (width 0.5) (layer "B.Cu") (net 1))
 (segment (start 163.5 106.775) (end 163.5 110.025) (width 0.5) (layer "B.Cu") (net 1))
 (segment (start 81.75 107.55) (end 81.75 111.399999) (width 0.5) (layer "B.Cu") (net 1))
 (segment (start 120.45 107.15) (end 120.45 111.549999) (width 0.5) (layer "B.Cu") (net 1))
 (segment (start 120.45 111.549999) (end 120.289999 111.71) (width 0.5) (layer "B.Cu") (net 1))
 (segment (start 172.8 113.85) (end 169.45 113.85) (width 0.5) (layer "B.Cu") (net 1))
 (segment (start 123.55 121.3) (end 122.5 121.3) (width 0.5) (layer "B.Cu") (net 1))
 (segment (start 163.85 112.8) (end 163.575 112.525) (width 0.5) (layer "B.Cu") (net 1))
 (segment (start 142.65 119.85) (end 142.2 119.85) (width 0.5) (layer "B.Cu") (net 1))
 (segment (start 172.441666 118.5) (end 170.791666 116.85) (width 0.5) (layer "F.Cu") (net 2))
 (segment (start 172.45 118.5) (end 172.441666 118.5) (width 0.5) (layer "F.Cu") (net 2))
 (segment (start 170.791666 115.891666) (end 170.791666 116.85) (width 0.25) (layer "F.Cu") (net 2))
 (segment (start 172.59 118.64) (end 172.45 118.5) (width 0.5) (layer "F.Cu") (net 2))
 (segment (start 172.59 120.475) (end 172.59 118.64) (width 0.5) (layer "F.Cu") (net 2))
 (via (at 170.791666 115.891666) (size 0.6) (drill 0.3) (layers "F.Cu" "B.Cu") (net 2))
 (segment (start 134.139999 106.760001) (end 134.139999 109.17) (width 0.25) (layer "B.Cu") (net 2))
 (segment (start 170.7 115.8) (end 163.369999 115.8) (width 0.25) (layer "B.Cu") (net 2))
 (segment (start 170.791666 115.891666) (end 170.7 115.8) (width 0.25) (layer "B.Cu") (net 2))
 (segment (start 163.369999 115.8) (end 152.569999 105) (width 0.25) (layer "B.Cu") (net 2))
 (segment (start 135.9 105) (end 134.139999 106.760001) (width 0.25) (layer "B.Cu") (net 2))
 (segment (start 152.569999 105) (end 135.9 105) (width 0.25) (layer "B.Cu") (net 2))
 (segment (start 165.225 117.65) (end 166.025 116.85) (width 0.25) (layer "F.Cu") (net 10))
 (segment (start 161.35 117.2) (end 161.8 117.65) (width 0.25) (layer "F.Cu") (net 10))
 (segment (start 161.8 117.65) (end 165.225 117.65) (width 0.25) (layer "F.Cu") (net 10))
 (segment (start 170.05 120.475) (end 166.425 116.85) (width 0.5) (layer "F.Cu") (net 10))
 (segment (start 166.425 116.85) (end 166.025 116.85) (width 0.5) (layer "F.Cu") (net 10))
 (via (at 161.35 117.2) (size 0.8) (drill 0.4) (layers "F.Cu" "B.Cu") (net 10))
 (segment (start 153.564999 109.414999) (end 153.564999 109.17) (width 0.25) (layer "B.Cu") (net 10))
 (segment (start 161.35 117.2) (end 153.564999 109.414999) (width 0.25) (layer "B.Cu") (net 10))
 (segment (start 175.13 120.475) (end 175.13 118.51) (width 0.5) (layer "F.Cu") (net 3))
 (segment (start 175.685 116.976668) (end 175.558332 116.85) (width 0.5) (layer "F.Cu") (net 3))
 (segment (start 175.5 116.791668) (end 175.558332 116.85) (width 0.25) (layer "F.Cu") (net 3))
 (segment (start 175.5 115.85) (end 175.5 116.791668) (width 0.25) (layer "F.Cu") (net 3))
 (segment (start 175.13 118.51) (end 175.685 117.955) (width 0.5) (layer "F.Cu") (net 3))
 (segment (start 175.685 117.955) (end 175.685 116.976668) (width 0.5) (layer "F.Cu") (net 3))
 (via (at 175.5 115.85) (size 0.8) (drill 0.4) (layers "F.Cu" "B.Cu") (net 3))
 (segment (start 114.714999 105.485001) (end 114.714999 109.17) (width 0.25) (layer "B.Cu") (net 3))
 (segment (start 175.5 115.85) (end 175.45 115.85) (width 0.25) (layer "B.Cu") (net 3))
 (segment (start 174.866666 115.266666) (end 170.532782 115.266666) (width 0.25) (layer "B.Cu") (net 3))
 (segment (start 170.499448 115.3) (end 164.25 115.3) (width 0.25) (layer "B.Cu") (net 3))
 (segment (start 170.532782 115.266666) (end 170.499448 115.3) (width 0.25) (layer "B.Cu") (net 3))
 (segment (start 164.25 115.3) (end 152.8 103.85) (width 0.25) (layer "B.Cu") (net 3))
 (segment (start 116.35 103.85) (end 114.714999 105.485001) (width 0.25) (layer "B.Cu") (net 3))
 (segment (start 152.8 103.85) (end 116.35 103.85) (width 0.25) (layer "B.Cu") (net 3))
 (segment (start 175.45 115.85) (end 174.866666 115.266666) (width 0.25) (layer "B.Cu") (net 3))
 (segment (start 179.5 115.1) (end 179.5 115.4) (width 0.25) (layer "F.Cu") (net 7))
 (segment (start 180.325 116.85) (end 179.4 117.775) (width 0.5) (layer "F.Cu") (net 7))
 (segment (start 179.5 115.4) (end 180.325 116.225) (width 0.25) (layer "F.Cu") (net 7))
 (segment (start 180.325 116.225) (end 180.325 116.85) (width 0.25) (layer "F.Cu") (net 7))
 (segment (start 177.67 118.73) (end 177.67 120.475) (width 0.5) (layer "F.Cu") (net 7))
 (segment (start 178.625 117.775) (end 177.67 118.73) (width 0.5) (layer "F.Cu") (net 7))
 (segment (start 179.4 117.775) (end 178.625 117.775) (width 0.5) (layer "F.Cu") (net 7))
 (via (at 179.5 115.1) (size 0.8) (drill 0.4) (layers "F.Cu" "B.Cu") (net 7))
 (segment (start 177 117.45) (end 176.05 118.4) (width 0.25) (layer "B.Cu") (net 7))
 (segment (start 97.2 121.35) (end 97.2 111.080001) (width 0.25) (layer "B.Cu") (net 7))
 (segment (start 97.2 111.080001) (end 95.289999 109.17) (width 0.25) (layer "B.Cu") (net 7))
 (segment (start 176.05 118.4) (end 159.25 118.4) (width 0.25) (layer "B.Cu") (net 7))
 (segment (start 177.7 115.2) (end 177.8 115.1) (width 0.25) (layer "B.Cu") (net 7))
 (segment (start 159.25 118.4) (end 155.25 122.4) (width 0.25) (layer "B.Cu") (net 7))
 (segment (start 177.8 115.1) (end 179.5 115.1) (width 0.25) (layer "B.Cu") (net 7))
 (segment (start 177 117.45) (end 177 115.9) (width 0.25) (layer "B.Cu") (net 7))
 (segment (start 177 115.9) (end 177.7 115.2) (width 0.25) (layer "B.Cu") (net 7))
 (segment (start 155.25 122.4) (end 98.25 122.4) (width 0.25) (layer "B.Cu") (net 7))
 (segment (start 98.25 122.4) (end 97.2 121.35) (width 0.25) (layer "B.Cu") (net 7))
 (segment (start 166.925 110.5) (end 166.525 110.1) (width 0.5) (layer "B.Cu") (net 12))
 (segment (start 177.35 110.1) (end 176.95 110.5) (width 0.5) (layer "B.Cu") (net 12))
 (segment (start 176.95 110.5) (end 166.925 110.5) (width 0.5) (layer "B.Cu") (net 12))
 (segment (start 132.175 117.15) (end 131 118.325) (width 0.5) (layer "F.Cu") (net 6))
 (segment (start 91.374999 118.7) (end 104.25 118.7) (width 0.5) (layer "F.Cu") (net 6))
 (segment (start 142.1 117.15) (end 132.175 117.15) (width 0.5) (layer "F.Cu") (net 6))
 (segment (start 90.649999 117.975) (end 91.374999 118.7) (width 0.5) (layer "F.Cu") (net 6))
 (segment (start 123.2 118.35) (end 123.15 118.4) (width 0.5) (layer "F.Cu") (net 6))
 (segment (start 150.7 118.15) (end 148.799999 118.15) (width 0.5) (layer "F.Cu") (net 6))
 (segment (start 123.15 118.4) (end 112.6 118.4) (width 0.5) (layer "F.Cu") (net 6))
 (segment (start 167.515 105.3) (end 154.665 118.15) (width 0.5) (layer "F.Cu") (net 6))
 (segment (start 110.554999 118.4) (end 112.6 118.4) (width 0.5) (layer "F.Cu") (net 6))
 (segment (start 131 118.325) (end 129.479999 118.325) (width 0.5) (layer "F.Cu") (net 6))
 (segment (start 154.665 118.15) (end 150.7 118.15) (width 0.5) (layer "F.Cu") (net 6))
 (via (at 142.1 117.15) (size 0.8) (drill 0.4) (layers "F.Cu" "B.Cu") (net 6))
 (via (at 112.6 118.4) (size 0.8) (drill 0.4) (layers "F.Cu" "B.Cu") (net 6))
 (via (at 123.2 118.35) (size 0.8) (drill 0.4) (layers "F.Cu" "B.Cu") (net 6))
 (via (at 131 118.325) (size 0.8) (drill 0.4) (layers "F.Cu" "B.Cu") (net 6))
 (via (at 104.25 118.7) (size 0.8) (drill 0.4) (layers "F.Cu" "B.Cu") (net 6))
 (via (at 150.7 118.15) (size 0.8) (drill 0.4) (layers "F.Cu" "B.Cu") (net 6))
 (segment (start 142.1 117.15) (end 143.1 118.15) (width 0.5) (layer "B.Cu") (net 6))
 (segment (start 123.2 118.35) (end 130.975 118.35) (width 0.5) (layer "B.Cu") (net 6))
 (segment (start 112.3 118.7) (end 112.6 118.4) (width 0.5) (layer "B.Cu") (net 6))
 (segment (start 143.1 118.15) (end 150.7 118.15) (width 0.5) (layer "B.Cu") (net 6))
 (segment (start 130.975 118.35) (end 131 118.325) (width 0.5) (layer "B.Cu") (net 6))
 (segment (start 104.25 118.7) (end 112.3 118.7) (width 0.5) (layer "B.Cu") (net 6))
 (segment (start 129.479999 120.075) (end 130.429999 119.125) (width 0.25) (layer "F.Cu") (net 5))
 (segment (start 130.429999 119.125) (end 144.724999 119.125) (width 0.25) (layer "F.Cu") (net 5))
 (segment (start 144.724999 119.125) (end 145.699999 118.15) (width 0.25) (layer "F.Cu") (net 5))
 (segment (start 149.374999 120.475) (end 162.43 120.475) (width 0.25) (layer "F.Cu") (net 9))
 (segment (start 148.799999 119.9) (end 149.374999 120.475) (width 0.25) (layer "F.Cu") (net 9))
 (segment (start 110.404999 120.15) (end 124.554999 120.15) (width 0.25) (layer "F.Cu") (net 4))
 (segment (start 124.554999 120.15) (end 126.379999 118.325) (width 0.25) (layer "F.Cu") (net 4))
 (segment (start 90.649999 119.725) (end 106.129999 119.725) (width 0.25) (layer "F.Cu") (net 8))
 (segment (start 106.129999 119.725) (end 107.454999 118.4) (width 0.25) (layer "F.Cu") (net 8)))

